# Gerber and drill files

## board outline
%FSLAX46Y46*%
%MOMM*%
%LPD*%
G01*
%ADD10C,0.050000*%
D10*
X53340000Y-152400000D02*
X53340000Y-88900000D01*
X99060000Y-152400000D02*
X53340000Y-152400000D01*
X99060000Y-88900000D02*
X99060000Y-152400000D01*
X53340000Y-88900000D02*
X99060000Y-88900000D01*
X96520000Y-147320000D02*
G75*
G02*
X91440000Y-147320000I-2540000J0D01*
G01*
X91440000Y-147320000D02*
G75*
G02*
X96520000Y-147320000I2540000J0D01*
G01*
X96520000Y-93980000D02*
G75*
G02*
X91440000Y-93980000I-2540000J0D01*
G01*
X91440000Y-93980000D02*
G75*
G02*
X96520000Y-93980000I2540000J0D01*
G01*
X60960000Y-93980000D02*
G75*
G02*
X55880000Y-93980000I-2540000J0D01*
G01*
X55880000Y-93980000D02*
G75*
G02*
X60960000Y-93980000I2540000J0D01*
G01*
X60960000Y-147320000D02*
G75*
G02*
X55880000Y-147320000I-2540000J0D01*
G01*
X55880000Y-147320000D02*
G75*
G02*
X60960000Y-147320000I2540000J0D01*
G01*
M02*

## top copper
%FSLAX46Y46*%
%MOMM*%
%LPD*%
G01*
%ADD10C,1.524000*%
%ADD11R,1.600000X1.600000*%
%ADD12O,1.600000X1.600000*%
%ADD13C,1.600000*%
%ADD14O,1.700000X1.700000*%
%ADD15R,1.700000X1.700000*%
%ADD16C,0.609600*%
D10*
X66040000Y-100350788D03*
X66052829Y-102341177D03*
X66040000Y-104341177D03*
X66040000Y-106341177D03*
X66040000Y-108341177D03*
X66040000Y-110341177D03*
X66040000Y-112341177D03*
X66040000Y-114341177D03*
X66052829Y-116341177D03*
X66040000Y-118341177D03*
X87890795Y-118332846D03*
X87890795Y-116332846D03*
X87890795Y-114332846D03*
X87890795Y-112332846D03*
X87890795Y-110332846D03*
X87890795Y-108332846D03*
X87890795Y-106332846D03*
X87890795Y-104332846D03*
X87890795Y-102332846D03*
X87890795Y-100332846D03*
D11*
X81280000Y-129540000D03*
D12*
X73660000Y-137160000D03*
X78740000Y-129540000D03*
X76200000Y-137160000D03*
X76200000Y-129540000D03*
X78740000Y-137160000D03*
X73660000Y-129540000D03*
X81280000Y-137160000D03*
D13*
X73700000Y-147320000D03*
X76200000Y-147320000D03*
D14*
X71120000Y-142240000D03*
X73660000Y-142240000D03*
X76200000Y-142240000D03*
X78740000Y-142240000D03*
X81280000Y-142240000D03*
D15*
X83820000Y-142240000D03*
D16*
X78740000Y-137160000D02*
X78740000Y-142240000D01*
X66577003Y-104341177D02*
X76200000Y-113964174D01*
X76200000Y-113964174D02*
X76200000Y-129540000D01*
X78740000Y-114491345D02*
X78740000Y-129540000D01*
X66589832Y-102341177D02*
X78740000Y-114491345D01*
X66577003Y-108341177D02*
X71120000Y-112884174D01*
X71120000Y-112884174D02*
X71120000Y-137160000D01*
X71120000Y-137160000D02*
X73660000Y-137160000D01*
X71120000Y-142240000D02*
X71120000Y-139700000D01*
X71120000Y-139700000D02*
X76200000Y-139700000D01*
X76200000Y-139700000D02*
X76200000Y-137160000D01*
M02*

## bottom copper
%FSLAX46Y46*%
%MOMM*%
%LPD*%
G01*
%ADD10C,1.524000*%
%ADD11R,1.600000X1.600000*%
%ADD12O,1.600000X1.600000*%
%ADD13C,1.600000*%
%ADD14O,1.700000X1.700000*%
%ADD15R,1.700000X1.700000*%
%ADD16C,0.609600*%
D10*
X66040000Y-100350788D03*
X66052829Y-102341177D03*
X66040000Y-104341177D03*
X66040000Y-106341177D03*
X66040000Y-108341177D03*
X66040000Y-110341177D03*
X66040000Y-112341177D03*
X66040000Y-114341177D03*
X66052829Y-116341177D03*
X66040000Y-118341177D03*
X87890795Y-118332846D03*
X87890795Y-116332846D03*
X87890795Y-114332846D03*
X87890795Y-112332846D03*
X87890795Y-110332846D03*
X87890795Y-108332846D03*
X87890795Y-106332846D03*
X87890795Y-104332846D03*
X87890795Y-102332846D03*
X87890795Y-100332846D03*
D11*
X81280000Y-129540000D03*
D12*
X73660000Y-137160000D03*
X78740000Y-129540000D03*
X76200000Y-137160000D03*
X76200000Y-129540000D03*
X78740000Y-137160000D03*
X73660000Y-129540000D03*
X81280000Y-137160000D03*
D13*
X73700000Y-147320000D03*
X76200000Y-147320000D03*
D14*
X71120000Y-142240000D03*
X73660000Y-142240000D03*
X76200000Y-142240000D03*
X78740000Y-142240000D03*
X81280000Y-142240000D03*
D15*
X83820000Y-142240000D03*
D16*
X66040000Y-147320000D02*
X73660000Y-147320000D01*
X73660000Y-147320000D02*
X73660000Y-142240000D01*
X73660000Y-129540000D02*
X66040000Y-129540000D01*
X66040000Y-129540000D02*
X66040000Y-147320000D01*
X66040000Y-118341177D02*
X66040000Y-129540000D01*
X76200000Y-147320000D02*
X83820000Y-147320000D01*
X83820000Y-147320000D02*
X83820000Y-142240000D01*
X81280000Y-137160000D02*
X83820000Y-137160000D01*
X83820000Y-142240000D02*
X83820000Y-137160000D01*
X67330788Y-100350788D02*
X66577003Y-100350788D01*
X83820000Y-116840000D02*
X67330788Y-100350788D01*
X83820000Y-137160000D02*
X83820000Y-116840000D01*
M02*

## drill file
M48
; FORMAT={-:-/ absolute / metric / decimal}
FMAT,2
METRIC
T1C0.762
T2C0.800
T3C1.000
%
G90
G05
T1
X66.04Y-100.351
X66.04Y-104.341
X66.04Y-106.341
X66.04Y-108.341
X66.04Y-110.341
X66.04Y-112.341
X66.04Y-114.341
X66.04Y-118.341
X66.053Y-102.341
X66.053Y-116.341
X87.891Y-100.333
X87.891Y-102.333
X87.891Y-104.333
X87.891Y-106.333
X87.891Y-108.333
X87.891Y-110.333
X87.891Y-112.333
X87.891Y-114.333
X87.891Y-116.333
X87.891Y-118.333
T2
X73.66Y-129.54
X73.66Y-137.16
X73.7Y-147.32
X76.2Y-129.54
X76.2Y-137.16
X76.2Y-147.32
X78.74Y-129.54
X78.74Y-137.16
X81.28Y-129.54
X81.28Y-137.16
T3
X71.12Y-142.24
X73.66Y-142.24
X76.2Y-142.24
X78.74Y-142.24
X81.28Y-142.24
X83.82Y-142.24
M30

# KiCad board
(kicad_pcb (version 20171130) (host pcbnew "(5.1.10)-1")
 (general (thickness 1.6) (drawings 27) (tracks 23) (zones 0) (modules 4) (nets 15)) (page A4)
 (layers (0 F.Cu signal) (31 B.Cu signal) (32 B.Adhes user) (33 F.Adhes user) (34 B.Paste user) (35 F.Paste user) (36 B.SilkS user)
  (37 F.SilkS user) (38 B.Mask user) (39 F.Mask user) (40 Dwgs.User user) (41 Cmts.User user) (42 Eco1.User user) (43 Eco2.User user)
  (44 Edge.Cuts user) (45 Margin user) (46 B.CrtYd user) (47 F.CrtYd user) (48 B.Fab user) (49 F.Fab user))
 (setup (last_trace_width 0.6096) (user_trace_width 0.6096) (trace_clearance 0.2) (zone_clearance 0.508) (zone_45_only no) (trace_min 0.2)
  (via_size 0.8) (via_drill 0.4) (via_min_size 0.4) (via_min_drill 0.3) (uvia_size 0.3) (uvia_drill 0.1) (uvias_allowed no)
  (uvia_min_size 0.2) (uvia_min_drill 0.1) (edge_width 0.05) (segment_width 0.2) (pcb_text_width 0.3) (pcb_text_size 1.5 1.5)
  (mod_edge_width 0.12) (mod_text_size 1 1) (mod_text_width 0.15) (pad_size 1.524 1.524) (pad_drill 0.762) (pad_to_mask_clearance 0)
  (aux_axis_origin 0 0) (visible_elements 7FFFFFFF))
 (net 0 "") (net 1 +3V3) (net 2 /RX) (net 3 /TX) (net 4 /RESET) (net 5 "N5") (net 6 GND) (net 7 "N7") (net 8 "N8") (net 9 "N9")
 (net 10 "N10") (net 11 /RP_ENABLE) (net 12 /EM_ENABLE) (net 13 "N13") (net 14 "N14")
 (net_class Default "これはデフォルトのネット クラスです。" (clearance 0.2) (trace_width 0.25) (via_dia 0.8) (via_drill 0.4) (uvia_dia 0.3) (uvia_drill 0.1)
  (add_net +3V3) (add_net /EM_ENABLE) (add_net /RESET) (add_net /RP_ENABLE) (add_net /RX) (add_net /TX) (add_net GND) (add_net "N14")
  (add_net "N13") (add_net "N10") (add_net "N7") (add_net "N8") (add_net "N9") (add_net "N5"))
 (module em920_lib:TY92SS (layer F.Cu) (at 64.794502 127)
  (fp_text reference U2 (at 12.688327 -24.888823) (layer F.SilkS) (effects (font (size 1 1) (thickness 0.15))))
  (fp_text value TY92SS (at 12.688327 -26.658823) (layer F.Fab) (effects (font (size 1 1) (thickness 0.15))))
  (pad 1 thru_hole circle (at 1.245498 -26.649212) (size 1.524 1.524) (drill 0.762) (layers *.Cu *.Mask) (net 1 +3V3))
  (pad 2 thru_hole circle (at 1.258327 -24.658823) (size 1.524 1.524) (drill 0.762) (layers *.Cu *.Mask) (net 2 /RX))
  (pad 3 thru_hole circle (at 1.245498 -22.658823) (size 1.524 1.524) (drill 0.762) (layers *.Cu *.Mask) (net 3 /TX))
  (pad 4 thru_hole circle (at 1.245498 -20.658823) (size 1.524 1.524) (drill 0.762) (layers *.Cu *.Mask))
  (pad 5 thru_hole circle (at 1.245498 -18.658823) (size 1.524 1.524) (drill 0.762) (layers *.Cu *.Mask) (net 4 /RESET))
  (pad 6 thru_hole circle (at 1.245498 -16.658823) (size 1.524 1.524) (drill 0.762) (layers *.Cu *.Mask))
  (pad 7 thru_hole circle (at 1.245498 -14.658823) (size 1.524 1.524) (drill 0.762) (layers *.Cu *.Mask))
  (pad 8 thru_hole circle (at 1.245498 -12.658823) (size 1.524 1.524) (drill 0.762) (layers *.Cu *.Mask))
  (pad 9 thru_hole circle (at 1.258327 -10.658823) (size 1.524 1.524) (drill 0.762) (layers *.Cu *.Mask) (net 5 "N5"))
  (pad 10 thru_hole circle (at 1.245498 -8.658823) (size 1.524 1.524) (drill 0.762) (layers *.Cu *.Mask) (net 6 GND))
  (pad 11 thru_hole circle (at 23.096293 -8.667154) (size 1.524 1.524) (drill 0.762) (layers *.Cu *.Mask))
  (pad 12 thru_hole circle (at 23.096293 -10.667154) (size 1.524 1.524) (drill 0.762) (layers *.Cu *.Mask) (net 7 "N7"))
  (pad 13 thru_hole circle (at 23.096293 -12.667154) (size 1.524 1.524) (drill 0.762) (layers *.Cu *.Mask) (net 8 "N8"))
  (pad 14 thru_hole circle (at 23.096293 -14.667154) (size 1.524 1.524) (drill 0.762) (layers *.Cu *.Mask))
  (pad 15 thru_hole circle (at 23.096293 -16.667154) (size 1.524 1.524) (drill 0.762) (layers *.Cu *.Mask))
  (pad 16 thru_hole circle (at 23.096293 -18.667154) (size 1.524 1.524) (drill 0.762) (layers *.Cu *.Mask) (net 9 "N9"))
  (pad 17 thru_hole circle (at 23.096293 -20.667154) (size 1.524 1.524) (drill 0.762) (layers *.Cu *.Mask))
  (pad 18 thru_hole circle (at 23.096293 -22.667154) (size 1.524 1.524) (drill 0.762) (layers *.Cu *.Mask))
  (pad 19 thru_hole circle (at 23.096293 -24.667154) (size 1.524 1.524) (drill 0.762) (layers *.Cu *.Mask))
  (pad 20 thru_hole circle (at 23.096293 -26.667154) (size 1.524 1.524) (drill 0.762) (layers *.Cu *.Mask)))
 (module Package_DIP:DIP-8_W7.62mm (layer F.Cu) (at 81.28 129.54 270)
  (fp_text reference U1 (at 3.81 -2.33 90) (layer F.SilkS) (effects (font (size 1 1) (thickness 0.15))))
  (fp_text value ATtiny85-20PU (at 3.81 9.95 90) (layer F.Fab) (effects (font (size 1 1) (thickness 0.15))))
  (pad 1 thru_hole rect (at 0 0 270) (size 1.6 1.6) (drill 0.8) (layers *.Cu *.Mask) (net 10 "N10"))
  (pad 5 thru_hole oval (at 7.62 7.62 270) (size 1.6 1.6) (drill 0.8) (layers *.Cu *.Mask) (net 4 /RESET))
  (pad 2 thru_hole oval (at 0 2.54 270) (size 1.6 1.6) (drill 0.8) (layers *.Cu *.Mask) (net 2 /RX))
  (pad 6 thru_hole oval (at 7.62 5.08 270) (size 1.6 1.6) (drill 0.8) (layers *.Cu *.Mask) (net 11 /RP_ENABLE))
  (pad 3 thru_hole oval (at 0 5.08 270) (size 1.6 1.6) (drill 0.8) (layers *.Cu *.Mask) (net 3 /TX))
  (pad 7 thru_hole oval (at 7.62 2.54 270) (size 1.6 1.6) (drill 0.8) (layers *.Cu *.Mask) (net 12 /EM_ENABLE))
  (pad 4 thru_hole oval (at 0 7.62 270) (size 1.6 1.6) (drill 0.8) (layers *.Cu *.Mask) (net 6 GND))
  (pad 8 thru_hole oval (at 7.62 0 270) (size 1.6 1.6) (drill 0.8) (layers *.Cu *.Mask) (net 1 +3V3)))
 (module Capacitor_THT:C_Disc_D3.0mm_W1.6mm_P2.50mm (layer F.Cu) (at 76.2 147.32 180)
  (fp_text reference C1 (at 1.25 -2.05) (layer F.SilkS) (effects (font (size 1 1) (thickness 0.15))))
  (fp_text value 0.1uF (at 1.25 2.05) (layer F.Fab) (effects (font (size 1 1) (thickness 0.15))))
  (pad 2 thru_hole circle (at 2.5 0 180) (size 1.6 1.6) (drill 0.8) (layers *.Cu *.Mask) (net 6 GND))
  (pad 1 thru_hole circle (at 0 0 180) (size 1.6 1.6) (drill 0.8) (layers *.Cu *.Mask) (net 1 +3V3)))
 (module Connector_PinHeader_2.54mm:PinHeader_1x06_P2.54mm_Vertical (layer F.Cu) (at 83.82 142.24 270)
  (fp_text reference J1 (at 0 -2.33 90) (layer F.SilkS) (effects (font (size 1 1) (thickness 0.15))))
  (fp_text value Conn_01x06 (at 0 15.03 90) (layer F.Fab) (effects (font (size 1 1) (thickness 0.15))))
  (pad 6 thru_hole oval (at 0 12.7 270) (size 1.7 1.7) (drill 1) (layers *.Cu *.Mask) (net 11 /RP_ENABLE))
  (pad 5 thru_hole oval (at 0 10.16 270) (size 1.7 1.7) (drill 1) (layers *.Cu *.Mask) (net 6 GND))
  (pad 4 thru_hole oval (at 0 7.62 270) (size 1.7 1.7) (drill 1) (layers *.Cu *.Mask) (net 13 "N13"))
  (pad 3 thru_hole oval (at 0 5.08 270) (size 1.7 1.7) (drill 1) (layers *.Cu *.Mask) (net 12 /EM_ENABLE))
  (pad 2 thru_hole oval (at 0 2.54 270) (size 1.7 1.7) (drill 1) (layers *.Cu *.Mask) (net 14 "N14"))
  (pad 1 thru_hole rect (at 0 0 270) (size 1.7 1.7) (drill 1) (layers *.Cu *.Mask) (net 1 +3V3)))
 (gr_line (start 53.34 152.4) (end 53.34 88.9) (layer Edge.Cuts) (width 0.05))
 (gr_line (start 99.06 152.4) (end 53.34 152.4) (layer Edge.Cuts) (width 0.05))
 (gr_line (start 99.06 88.9) (end 99.06 152.4) (layer Edge.Cuts) (width 0.05))
 (gr_line (start 53.34 88.9) (end 99.06 88.9) (layer Edge.Cuts) (width 0.05))
 (gr_circle (center 93.98 147.32) (end 93.98 144.78) (layer Edge.Cuts) (width 0.05))
 (gr_circle (center 93.98 93.98) (end 93.98 96.52) (layer Edge.Cuts) (width 0.05))
 (gr_circle (center 58.42 93.98) (end 58.42 96.52) (layer Edge.Cuts) (width 0.05))
 (gr_circle (center 58.42 147.32) (end 60.96 147.32) (layer Edge.Cuts) (width 0.05))
 (segment (start 66.04 147.32) (end 73.66 147.32) (width 0.6096) (layer B.Cu) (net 6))
 (segment (start 73.66 147.32) (end 73.66 142.24) (width 0.6096) (layer B.Cu) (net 6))
 (segment (start 73.66 129.54) (end 66.04 129.54) (width 0.6096) (layer B.Cu) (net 6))
 (segment (start 66.04 129.54) (end 66.04 147.32) (width 0.6096) (layer B.Cu) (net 6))
 (segment (start 66.04 118.341177) (end 66.04 129.54) (width 0.6096) (layer B.Cu) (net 6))
 (segment (start 78.74 137.16) (end 78.74 142.24) (width 0.6096) (layer F.Cu) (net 12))
 (segment (start 76.2 147.32) (end 83.82 147.32) (width 0.6096) (layer B.Cu) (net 1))
 (segment (start 83.82 147.32) (end 83.82 142.24) (width 0.6096) (layer B.Cu) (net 1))
 (segment (start 81.28 137.16) (end 83.82 137.16) (width 0.6096) (layer B.Cu) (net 1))
 (segment (start 83.82 142.24) (end 83.82 137.16) (width 0.6096) (layer B.Cu) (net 1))
 (segment (start 67.330788 100.350788) (end 66.577003 100.350788) (width 0.6096) (layer B.Cu) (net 1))
 (segment (start 83.82 116.84) (end 67.330788 100.350788) (width 0.6096) (layer B.Cu) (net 1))
 (segment (start 83.82 137.16) (end 83.82 116.84) (width 0.6096) (layer B.Cu) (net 1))
 (segment (start 66.577003 104.341177) (end 76.2 113.964174) (width 0.6096) (layer F.Cu) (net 3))
 (segment (start 76.2 113.964174) (end 76.2 129.54) (width 0.6096) (layer F.Cu) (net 3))
 (segment (start 78.74 114.491345) (end 78.74 129.54) (width 0.6096) (layer F.Cu) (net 2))
 (segment (start 66.589832 102.341177) (end 78.74 114.491345) (width 0.6096) (layer F.Cu) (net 2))
 (segment (start 66.577003 108.341177) (end 71.12 112.884174) (width 0.6096) (layer F.Cu) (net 4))
 (segment (start 71.12 112.884174) (end 71.12 137.16) (width 0.6096) (layer F.Cu) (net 4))
 (segment (start 71.12 137.16) (end 73.66 137.16) (width 0.6096) (layer F.Cu) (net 4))
 (segment (start 71.12 142.24) (end 71.12 139.7) (width 0.6096) (layer F.Cu) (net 11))
 (segment (start 71.12 139.7) (end 76.2 139.7) (width 0.6096) (layer F.Cu) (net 11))
 (segment (start 76.2 139.7) (end 76.2 137.16) (width 0.6096) (layer F.Cu) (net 11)))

